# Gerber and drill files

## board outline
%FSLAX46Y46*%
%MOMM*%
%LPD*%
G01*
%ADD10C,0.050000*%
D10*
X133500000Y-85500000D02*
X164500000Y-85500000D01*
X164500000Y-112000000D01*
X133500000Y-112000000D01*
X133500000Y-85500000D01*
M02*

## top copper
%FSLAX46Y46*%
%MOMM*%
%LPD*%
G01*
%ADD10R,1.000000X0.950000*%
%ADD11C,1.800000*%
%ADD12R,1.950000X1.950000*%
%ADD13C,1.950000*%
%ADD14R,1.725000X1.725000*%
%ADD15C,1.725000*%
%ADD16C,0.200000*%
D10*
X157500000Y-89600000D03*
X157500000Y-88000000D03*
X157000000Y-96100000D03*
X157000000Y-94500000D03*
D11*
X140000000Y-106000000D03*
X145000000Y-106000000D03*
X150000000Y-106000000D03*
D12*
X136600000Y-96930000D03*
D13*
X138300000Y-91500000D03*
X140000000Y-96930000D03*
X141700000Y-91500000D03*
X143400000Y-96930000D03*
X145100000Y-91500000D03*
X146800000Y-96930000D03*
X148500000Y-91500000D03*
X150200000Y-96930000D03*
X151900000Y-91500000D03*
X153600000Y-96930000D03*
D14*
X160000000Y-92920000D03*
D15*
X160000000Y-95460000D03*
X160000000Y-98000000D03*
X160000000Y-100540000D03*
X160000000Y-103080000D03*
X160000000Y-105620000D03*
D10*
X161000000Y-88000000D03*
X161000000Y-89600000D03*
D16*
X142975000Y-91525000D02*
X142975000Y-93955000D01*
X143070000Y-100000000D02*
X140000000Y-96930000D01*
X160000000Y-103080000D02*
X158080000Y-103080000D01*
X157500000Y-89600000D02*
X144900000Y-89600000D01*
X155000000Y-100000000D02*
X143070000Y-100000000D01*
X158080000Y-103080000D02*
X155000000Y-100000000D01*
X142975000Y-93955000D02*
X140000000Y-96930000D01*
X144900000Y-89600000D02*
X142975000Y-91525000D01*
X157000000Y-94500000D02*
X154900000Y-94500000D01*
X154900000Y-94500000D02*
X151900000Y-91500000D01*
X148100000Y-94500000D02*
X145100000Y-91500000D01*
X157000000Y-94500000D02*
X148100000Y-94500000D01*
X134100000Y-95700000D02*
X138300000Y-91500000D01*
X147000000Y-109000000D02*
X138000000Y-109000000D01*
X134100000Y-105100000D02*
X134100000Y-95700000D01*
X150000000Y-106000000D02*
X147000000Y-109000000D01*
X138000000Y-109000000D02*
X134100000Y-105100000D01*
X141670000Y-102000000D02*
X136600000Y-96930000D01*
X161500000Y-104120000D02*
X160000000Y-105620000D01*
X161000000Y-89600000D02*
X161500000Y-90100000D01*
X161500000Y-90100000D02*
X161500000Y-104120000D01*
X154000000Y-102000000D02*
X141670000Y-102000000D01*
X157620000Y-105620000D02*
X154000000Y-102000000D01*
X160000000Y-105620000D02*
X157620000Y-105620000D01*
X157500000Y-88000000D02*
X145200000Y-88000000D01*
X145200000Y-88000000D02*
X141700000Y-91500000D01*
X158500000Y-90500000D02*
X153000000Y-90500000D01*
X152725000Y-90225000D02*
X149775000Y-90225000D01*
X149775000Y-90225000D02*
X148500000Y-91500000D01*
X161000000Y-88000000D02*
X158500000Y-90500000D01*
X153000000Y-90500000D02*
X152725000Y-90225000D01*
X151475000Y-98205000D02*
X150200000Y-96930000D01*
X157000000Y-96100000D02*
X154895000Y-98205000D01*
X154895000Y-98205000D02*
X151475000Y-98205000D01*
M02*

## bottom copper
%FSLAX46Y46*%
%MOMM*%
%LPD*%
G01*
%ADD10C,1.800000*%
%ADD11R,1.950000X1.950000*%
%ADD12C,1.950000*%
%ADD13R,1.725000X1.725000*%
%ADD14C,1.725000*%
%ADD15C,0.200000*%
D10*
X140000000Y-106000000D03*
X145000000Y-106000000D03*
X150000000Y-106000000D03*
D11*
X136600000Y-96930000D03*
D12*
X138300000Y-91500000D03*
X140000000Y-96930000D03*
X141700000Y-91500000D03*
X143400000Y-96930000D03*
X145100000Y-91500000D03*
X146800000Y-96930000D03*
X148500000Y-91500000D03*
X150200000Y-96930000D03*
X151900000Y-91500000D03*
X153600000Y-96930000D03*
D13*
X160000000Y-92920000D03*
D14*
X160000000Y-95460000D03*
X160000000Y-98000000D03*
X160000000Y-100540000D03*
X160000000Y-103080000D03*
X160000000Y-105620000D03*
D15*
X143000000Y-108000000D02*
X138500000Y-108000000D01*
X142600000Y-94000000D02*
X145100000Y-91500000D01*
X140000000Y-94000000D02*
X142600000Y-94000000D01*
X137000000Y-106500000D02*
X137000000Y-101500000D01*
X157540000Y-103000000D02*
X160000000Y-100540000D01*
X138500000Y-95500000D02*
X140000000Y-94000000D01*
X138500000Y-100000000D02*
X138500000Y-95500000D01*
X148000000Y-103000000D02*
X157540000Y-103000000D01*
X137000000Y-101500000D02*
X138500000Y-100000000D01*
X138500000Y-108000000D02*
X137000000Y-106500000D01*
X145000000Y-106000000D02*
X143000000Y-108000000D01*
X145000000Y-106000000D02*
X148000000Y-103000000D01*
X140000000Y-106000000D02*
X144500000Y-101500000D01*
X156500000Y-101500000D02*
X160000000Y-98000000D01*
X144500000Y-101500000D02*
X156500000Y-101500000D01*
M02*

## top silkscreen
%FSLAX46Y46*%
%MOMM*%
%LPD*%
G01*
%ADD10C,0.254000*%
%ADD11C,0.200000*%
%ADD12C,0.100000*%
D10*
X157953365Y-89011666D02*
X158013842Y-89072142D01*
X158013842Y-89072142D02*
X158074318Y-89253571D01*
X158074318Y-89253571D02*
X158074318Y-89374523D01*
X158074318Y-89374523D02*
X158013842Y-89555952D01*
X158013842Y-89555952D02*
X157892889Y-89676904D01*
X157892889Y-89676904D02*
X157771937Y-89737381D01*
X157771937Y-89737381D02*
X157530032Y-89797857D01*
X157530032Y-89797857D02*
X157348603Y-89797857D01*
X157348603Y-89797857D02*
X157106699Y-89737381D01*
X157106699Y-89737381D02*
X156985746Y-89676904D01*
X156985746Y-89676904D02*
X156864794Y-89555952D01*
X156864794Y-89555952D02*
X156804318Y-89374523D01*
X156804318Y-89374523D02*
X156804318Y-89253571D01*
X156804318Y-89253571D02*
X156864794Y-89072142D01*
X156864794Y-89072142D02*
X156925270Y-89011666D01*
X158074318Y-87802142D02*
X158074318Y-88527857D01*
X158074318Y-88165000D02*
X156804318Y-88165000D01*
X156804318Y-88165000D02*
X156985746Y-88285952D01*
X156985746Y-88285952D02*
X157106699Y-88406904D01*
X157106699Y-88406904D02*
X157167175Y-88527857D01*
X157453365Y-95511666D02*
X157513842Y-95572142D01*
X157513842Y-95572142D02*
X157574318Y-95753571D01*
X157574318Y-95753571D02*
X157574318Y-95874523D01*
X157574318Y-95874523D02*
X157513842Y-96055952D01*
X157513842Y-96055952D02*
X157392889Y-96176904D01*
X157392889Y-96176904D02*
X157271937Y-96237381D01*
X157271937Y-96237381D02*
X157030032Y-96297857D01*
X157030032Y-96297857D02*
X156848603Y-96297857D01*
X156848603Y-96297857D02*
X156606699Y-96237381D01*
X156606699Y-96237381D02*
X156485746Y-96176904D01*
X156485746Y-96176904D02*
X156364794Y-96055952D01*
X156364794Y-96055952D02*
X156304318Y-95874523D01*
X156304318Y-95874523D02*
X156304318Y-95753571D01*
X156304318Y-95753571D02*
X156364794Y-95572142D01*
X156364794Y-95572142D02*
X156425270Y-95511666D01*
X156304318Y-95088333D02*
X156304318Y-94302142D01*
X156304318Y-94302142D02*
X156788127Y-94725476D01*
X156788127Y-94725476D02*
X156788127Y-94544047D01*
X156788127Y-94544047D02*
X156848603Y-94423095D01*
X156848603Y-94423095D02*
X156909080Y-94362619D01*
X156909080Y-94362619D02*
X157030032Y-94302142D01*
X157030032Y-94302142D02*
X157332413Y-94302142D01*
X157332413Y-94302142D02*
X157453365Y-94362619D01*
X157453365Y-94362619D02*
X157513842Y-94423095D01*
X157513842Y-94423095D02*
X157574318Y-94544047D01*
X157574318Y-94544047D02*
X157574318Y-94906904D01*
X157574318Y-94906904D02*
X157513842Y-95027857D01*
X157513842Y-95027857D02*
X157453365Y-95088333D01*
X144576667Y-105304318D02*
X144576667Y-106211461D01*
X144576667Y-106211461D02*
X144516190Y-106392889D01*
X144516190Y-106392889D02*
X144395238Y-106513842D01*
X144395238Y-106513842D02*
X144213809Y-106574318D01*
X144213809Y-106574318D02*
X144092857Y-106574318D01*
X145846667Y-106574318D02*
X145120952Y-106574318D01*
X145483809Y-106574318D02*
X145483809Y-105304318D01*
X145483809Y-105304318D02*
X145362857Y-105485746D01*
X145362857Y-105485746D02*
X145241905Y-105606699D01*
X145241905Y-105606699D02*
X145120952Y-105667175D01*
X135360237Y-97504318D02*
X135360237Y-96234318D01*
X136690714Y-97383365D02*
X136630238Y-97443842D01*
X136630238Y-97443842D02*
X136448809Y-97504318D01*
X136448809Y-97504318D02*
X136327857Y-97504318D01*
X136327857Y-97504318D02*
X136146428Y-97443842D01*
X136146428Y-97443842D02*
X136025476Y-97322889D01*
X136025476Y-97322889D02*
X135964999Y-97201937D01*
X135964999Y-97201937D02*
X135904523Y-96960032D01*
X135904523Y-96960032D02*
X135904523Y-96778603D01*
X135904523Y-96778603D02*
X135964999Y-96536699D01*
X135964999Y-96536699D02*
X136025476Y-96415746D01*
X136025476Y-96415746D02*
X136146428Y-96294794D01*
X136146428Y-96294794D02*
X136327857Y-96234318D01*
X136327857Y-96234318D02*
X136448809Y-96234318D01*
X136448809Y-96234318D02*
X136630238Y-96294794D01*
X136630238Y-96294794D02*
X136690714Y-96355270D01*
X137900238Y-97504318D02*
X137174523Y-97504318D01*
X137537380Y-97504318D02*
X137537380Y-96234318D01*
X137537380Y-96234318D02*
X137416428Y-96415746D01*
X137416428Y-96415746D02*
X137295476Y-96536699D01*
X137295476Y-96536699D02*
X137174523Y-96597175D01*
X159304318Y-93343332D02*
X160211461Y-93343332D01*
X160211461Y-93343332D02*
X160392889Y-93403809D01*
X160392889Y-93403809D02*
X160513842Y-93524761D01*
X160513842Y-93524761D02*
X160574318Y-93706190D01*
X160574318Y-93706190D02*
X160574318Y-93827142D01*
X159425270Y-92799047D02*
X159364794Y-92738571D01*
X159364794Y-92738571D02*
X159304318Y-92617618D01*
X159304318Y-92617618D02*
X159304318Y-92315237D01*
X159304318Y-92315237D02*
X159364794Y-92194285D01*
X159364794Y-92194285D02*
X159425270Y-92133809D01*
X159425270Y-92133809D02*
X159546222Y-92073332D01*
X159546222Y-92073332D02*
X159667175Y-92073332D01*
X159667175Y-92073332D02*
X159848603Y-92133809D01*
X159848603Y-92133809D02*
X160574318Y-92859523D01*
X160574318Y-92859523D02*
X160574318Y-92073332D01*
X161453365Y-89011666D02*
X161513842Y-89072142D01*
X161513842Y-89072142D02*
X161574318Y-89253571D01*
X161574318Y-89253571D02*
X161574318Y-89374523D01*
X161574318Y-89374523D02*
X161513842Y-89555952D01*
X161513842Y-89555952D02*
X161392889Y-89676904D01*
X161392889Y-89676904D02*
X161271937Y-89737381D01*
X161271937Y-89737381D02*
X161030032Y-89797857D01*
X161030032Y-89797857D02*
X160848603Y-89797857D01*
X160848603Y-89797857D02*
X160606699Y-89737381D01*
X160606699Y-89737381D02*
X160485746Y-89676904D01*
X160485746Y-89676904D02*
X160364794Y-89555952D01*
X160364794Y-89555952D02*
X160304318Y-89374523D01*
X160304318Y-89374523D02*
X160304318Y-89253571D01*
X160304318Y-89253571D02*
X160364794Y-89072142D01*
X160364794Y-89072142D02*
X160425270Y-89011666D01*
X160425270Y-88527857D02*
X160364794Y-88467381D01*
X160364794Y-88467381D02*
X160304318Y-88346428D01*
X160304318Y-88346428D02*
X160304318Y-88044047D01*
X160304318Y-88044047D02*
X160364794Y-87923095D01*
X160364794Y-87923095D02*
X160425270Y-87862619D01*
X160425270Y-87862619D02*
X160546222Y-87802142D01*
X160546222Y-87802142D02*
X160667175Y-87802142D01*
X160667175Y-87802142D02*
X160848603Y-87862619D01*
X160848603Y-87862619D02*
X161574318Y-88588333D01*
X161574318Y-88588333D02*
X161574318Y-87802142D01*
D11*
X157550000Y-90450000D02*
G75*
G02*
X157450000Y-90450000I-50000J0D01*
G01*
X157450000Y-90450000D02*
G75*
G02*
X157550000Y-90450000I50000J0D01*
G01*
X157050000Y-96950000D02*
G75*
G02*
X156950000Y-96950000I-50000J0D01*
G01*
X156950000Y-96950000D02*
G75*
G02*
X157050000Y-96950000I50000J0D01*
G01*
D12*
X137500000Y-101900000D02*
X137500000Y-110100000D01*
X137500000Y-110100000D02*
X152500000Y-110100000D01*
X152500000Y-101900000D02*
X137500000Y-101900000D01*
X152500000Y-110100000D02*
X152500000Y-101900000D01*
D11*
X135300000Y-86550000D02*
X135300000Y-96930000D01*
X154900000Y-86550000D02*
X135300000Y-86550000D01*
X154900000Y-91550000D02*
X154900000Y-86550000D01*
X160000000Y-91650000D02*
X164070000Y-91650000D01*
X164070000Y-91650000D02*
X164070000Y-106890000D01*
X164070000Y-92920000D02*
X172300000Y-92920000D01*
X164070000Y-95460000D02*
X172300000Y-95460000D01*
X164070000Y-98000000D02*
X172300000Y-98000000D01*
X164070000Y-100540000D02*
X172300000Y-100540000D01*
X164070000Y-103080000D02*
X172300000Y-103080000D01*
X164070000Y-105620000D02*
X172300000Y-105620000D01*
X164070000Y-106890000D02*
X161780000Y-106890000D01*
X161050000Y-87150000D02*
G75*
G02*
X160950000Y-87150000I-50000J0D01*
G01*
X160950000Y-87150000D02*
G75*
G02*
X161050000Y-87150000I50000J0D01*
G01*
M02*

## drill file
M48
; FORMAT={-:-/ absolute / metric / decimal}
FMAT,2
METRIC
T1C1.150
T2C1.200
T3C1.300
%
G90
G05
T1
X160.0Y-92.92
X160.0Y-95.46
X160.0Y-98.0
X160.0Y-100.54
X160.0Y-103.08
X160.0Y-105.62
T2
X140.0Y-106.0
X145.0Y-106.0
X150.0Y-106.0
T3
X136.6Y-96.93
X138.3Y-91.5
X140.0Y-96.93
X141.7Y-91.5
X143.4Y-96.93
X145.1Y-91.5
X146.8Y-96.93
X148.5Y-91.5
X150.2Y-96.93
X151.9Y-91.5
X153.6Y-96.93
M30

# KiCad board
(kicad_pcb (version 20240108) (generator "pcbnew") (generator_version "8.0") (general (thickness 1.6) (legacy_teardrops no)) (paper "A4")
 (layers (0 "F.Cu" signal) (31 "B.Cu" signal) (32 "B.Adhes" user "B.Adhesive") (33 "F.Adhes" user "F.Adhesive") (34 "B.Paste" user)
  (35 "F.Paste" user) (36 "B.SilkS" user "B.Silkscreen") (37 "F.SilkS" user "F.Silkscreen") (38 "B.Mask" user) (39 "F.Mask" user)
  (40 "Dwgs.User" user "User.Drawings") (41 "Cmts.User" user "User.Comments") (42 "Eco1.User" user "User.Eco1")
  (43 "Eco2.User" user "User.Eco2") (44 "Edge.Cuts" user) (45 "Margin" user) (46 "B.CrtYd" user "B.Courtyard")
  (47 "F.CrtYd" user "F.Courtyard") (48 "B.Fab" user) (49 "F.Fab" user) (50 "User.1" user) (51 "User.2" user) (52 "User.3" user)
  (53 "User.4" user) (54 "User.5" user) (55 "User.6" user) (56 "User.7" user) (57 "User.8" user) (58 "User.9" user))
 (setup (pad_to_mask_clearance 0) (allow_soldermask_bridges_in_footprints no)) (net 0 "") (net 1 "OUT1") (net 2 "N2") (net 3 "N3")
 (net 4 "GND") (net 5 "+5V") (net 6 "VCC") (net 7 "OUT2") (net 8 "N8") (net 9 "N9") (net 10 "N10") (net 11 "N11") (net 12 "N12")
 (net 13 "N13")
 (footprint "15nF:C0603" (layer "F.Cu") (at 157.5 88.8 90)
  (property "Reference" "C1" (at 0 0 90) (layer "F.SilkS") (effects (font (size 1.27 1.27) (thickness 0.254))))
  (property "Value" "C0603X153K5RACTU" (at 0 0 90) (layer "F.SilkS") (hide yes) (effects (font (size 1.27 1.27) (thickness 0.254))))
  (fp_circle (center -1.65 0) (end -1.65 0.05) (stroke (width 0.2) (type solid)) (fill none) (layer "F.SilkS"))
  (pad "1" smd rect (at -0.8 0 90) (size 0.95 1) (layers "F.Cu" "F.Paste" "F.Mask") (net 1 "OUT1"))
  (pad "2" smd rect (at 0.8 0 90) (size 0.95 1) (layers "F.Cu" "F.Paste" "F.Mask") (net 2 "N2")))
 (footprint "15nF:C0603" (layer "F.Cu") (at 157 95.3 90)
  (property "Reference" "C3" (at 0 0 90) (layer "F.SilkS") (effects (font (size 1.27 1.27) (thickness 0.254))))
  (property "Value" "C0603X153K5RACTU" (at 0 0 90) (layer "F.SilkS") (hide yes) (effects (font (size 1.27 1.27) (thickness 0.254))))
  (fp_circle (center -1.65 0) (end -1.65 0.05) (stroke (width 0.2) (type solid)) (fill none) (layer "F.SilkS"))
  (pad "1" smd rect (at -0.8 0 90) (size 0.95 1) (layers "F.Cu" "F.Paste" "F.Mask") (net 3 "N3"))
  (pad "2" smd rect (at 0.8 0 90) (size 0.95 1) (layers "F.Cu" "F.Paste" "F.Mask") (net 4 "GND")))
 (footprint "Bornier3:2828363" (layer "F.Cu") (at 140 106)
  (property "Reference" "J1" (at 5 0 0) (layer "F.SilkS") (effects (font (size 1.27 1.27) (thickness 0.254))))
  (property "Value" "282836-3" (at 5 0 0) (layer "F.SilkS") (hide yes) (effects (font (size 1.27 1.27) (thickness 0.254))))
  (fp_line (start -2.5 -4.1) (end -2.5 4.1) (stroke (width 0.1) (type solid)) (layer "F.SilkS"))
  (fp_line (start -2.5 4.1) (end 12.5 4.1) (stroke (width 0.1) (type solid)) (layer "F.SilkS"))
  (fp_line (start 12.5 -4.1) (end -2.5 -4.1) (stroke (width 0.1) (type solid)) (layer "F.SilkS"))
  (fp_line (start 12.5 4.1) (end 12.5 -4.1) (stroke (width 0.1) (type solid)) (layer "F.SilkS"))
  (pad "1" thru_hole circle (at 0 0) (size 1.8 1.8) (drill 1.2) (layers "*.Cu" "*.Mask") (remove_unused_layers no) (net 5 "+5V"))
  (pad "2" thru_hole circle (at 5 0) (size 1.8 1.8) (drill 1.2) (layers "*.Cu" "*.Mask") (remove_unused_layers no) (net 4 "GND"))
  (pad "3" thru_hole circle (at 10 0) (size 1.8 1.8) (drill 1.2) (layers "*.Cu" "*.Mask") (remove_unused_layers no) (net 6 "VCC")))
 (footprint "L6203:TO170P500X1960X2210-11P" (layer "F.Cu") (at 136.6 96.93)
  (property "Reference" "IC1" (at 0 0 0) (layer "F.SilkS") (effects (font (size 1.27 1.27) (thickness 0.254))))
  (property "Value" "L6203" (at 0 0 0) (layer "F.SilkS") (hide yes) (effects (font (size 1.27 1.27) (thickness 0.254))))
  (fp_line (start -1.3 -10.38) (end -1.3 0) (stroke (width 0.2) (type solid)) (layer "F.SilkS"))
  (fp_line (start 18.3 -10.38) (end -1.3 -10.38) (stroke (width 0.2) (type solid)) (layer "F.SilkS"))
  (fp_line (start 18.3 -5.38) (end 18.3 -10.38) (stroke (width 0.2) (type solid)) (layer "F.SilkS"))
  (pad "1" thru_hole rect (at 0 0) (size 1.95 1.95) (drill 1.3) (layers "*.Cu" "*.Mask") (remove_unused_layers no) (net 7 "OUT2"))
  (pad "2" thru_hole circle (at 1.7 -5.43) (size 1.95 1.95) (drill 1.3) (layers "*.Cu" "*.Mask") (remove_unused_layers no) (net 6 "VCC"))
  (pad "3" thru_hole circle (at 3.4 0) (size 1.95 1.95) (drill 1.3) (layers "*.Cu" "*.Mask") (remove_unused_layers no) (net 1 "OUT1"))
  (pad "4" thru_hole circle (at 5.1 -5.43) (size 1.95 1.95) (drill 1.3) (layers "*.Cu" "*.Mask") (remove_unused_layers no) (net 2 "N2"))
  (pad "5" thru_hole circle (at 6.8 0) (size 1.95 1.95) (drill 1.3) (layers "*.Cu" "*.Mask") (remove_unused_layers no) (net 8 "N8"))
  (pad "6" thru_hole circle (at 8.5 -5.43) (size 1.95 1.95) (drill 1.3) (layers "*.Cu" "*.Mask") (remove_unused_layers no) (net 4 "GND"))
  (pad "7" thru_hole circle (at 10.2 0) (size 1.95 1.95) (drill 1.3) (layers "*.Cu" "*.Mask") (remove_unused_layers no) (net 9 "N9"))
  (pad "8" thru_hole circle (at 11.9 -5.43) (size 1.95 1.95) (drill 1.3) (layers "*.Cu" "*.Mask") (remove_unused_layers no) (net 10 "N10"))
  (pad "9" thru_hole circle (at 13.6 0) (size 1.95 1.95) (drill 1.3) (layers "*.Cu" "*.Mask") (remove_unused_layers no) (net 3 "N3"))
  (pad "10" thru_hole circle (at 15.3 -5.43) (size 1.95 1.95) (drill 1.3) (layers "*.Cu" "*.Mask") (remove_unused_layers no) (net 4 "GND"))
  (pad "11" thru_hole circle (at 17 0) (size 1.95 1.95) (drill 1.3) (layers "*.Cu" "*.Mask") (remove_unused_layers no) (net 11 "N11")))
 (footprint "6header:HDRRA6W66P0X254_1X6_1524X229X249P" (layer "F.Cu") (at 160 92.92 -90)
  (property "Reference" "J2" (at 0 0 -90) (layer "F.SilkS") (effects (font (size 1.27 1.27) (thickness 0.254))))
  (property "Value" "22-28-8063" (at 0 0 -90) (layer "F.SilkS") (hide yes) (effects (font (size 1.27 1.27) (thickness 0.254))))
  (fp_line (start -1.27 0) (end -1.27 -4.07) (stroke (width 0.2) (type solid)) (layer "F.SilkS"))
  (fp_line (start -1.27 -4.07) (end 13.97 -4.07) (stroke (width 0.2) (type solid)) (layer "F.SilkS"))
  (fp_line (start 0 -4.07) (end 0 -12.3) (stroke (width 0.2) (type solid)) (layer "F.SilkS"))
  (fp_line (start 2.54 -4.07) (end 2.54 -12.3) (stroke (width 0.2) (type solid)) (layer "F.SilkS"))
  (fp_line (start 5.08 -4.07) (end 5.08 -12.3) (stroke (width 0.2) (type solid)) (layer "F.SilkS"))
  (fp_line (start 7.62 -4.07) (end 7.62 -12.3) (stroke (width 0.2) (type solid)) (layer "F.SilkS"))
  (fp_line (start 10.16 -4.07) (end 10.16 -12.3) (stroke (width 0.2) (type solid)) (layer "F.SilkS"))
  (fp_line (start 12.7 -4.07) (end 12.7 -12.3) (stroke (width 0.2) (type solid)) (layer "F.SilkS"))
  (fp_line (start 13.97 -4.07) (end 13.97 -1.78) (stroke (width 0.2) (type solid)) (layer "F.SilkS"))
  (pad "1" thru_hole rect (at 0 0 270) (size 1.725 1.725) (drill 1.15) (layers "*.Cu" "*.Mask") (remove_unused_layers no) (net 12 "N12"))
  (pad "2" thru_hole circle (at 2.54 0 270) (size 1.725 1.725) (drill 1.15) (layers "*.Cu" "*.Mask") (remove_unused_layers no)
   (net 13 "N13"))
  (pad "3" thru_hole circle (at 5.08 0 270) (size 1.725 1.725) (drill 1.15) (layers "*.Cu" "*.Mask") (remove_unused_layers no) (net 5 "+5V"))
  (pad "4" thru_hole circle (at 7.62 0 270) (size 1.725 1.725) (drill 1.15) (layers "*.Cu" "*.Mask") (remove_unused_layers no) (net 4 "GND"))
  (pad "5" thru_hole circle (at 10.16 0 270) (size 1.725 1.725) (drill 1.15) (layers "*.Cu" "*.Mask") (remove_unused_layers no)
   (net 1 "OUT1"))
  (pad "6" thru_hole circle (at 12.7 0 270) (size 1.725 1.725) (drill 1.15) (layers "*.Cu" "*.Mask") (remove_unused_layers no)
   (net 7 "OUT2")))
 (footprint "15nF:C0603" (layer "F.Cu") (at 161 88.8 -90)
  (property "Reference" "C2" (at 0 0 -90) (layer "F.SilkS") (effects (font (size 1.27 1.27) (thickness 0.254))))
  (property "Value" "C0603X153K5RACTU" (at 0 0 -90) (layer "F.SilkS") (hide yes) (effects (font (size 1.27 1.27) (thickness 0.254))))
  (fp_circle (center -1.65 0) (end -1.65 0.05) (stroke (width 0.2) (type solid)) (fill none) (layer "F.SilkS"))
  (pad "1" smd rect (at -0.8 0 270) (size 0.95 1) (layers "F.Cu" "F.Paste" "F.Mask") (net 10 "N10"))
  (pad "2" smd rect (at 0.8 0 270) (size 0.95 1) (layers "F.Cu" "F.Paste" "F.Mask") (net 7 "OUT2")))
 (gr_rect (start 133.5 85.5) (end 164.5 112) (stroke (width 0.05) (type default)) (fill none) (layer "Edge.Cuts"))
 (segment (start 142.975 91.525) (end 142.975 93.955) (width 0.2) (layer "F.Cu") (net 1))
 (segment (start 143.07 100) (end 140 96.93) (width 0.2) (layer "F.Cu") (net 1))
 (segment (start 160 103.08) (end 158.08 103.08) (width 0.2) (layer "F.Cu") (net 1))
 (segment (start 157.5 89.6) (end 144.9 89.6) (width 0.2) (layer "F.Cu") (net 1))
 (segment (start 155 100) (end 143.07 100) (width 0.2) (layer "F.Cu") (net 1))
 (segment (start 158.08 103.08) (end 155 100) (width 0.2) (layer "F.Cu") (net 1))
 (segment (start 142.975 93.955) (end 140 96.93) (width 0.2) (layer "F.Cu") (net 1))
 (segment (start 144.9 89.6) (end 142.975 91.525) (width 0.2) (layer "F.Cu") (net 1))
 (segment (start 157 94.5) (end 154.9 94.5) (width 0.2) (layer "F.Cu") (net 4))
 (segment (start 154.9 94.5) (end 151.9 91.5) (width 0.2) (layer "F.Cu") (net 4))
 (segment (start 148.1 94.5) (end 145.1 91.5) (width 0.2) (layer "F.Cu") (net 4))
 (segment (start 157 94.5) (end 148.1 94.5) (width 0.2) (layer "F.Cu") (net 4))
 (segment (start 143 108) (end 138.5 108) (width 0.2) (layer "B.Cu") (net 4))
 (segment (start 142.6 94) (end 145.1 91.5) (width 0.2) (layer "B.Cu") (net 4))
 (segment (start 140 94) (end 142.6 94) (width 0.2) (layer "B.Cu") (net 4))
 (segment (start 137 106.5) (end 137 101.5) (width 0.2) (layer "B.Cu") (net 4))
 (segment (start 157.54 103) (end 160 100.54) (width 0.2) (layer "B.Cu") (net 4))
 (segment (start 138.5 95.5) (end 140 94) (width 0.2) (layer "B.Cu") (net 4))
 (segment (start 138.5 100) (end 138.5 95.5) (width 0.2) (layer "B.Cu") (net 4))
 (segment (start 148 103) (end 157.54 103) (width 0.2) (layer "B.Cu") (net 4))
 (segment (start 137 101.5) (end 138.5 100) (width 0.2) (layer "B.Cu") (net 4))
 (segment (start 138.5 108) (end 137 106.5) (width 0.2) (layer "B.Cu") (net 4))
 (segment (start 145 106) (end 143 108) (width 0.2) (layer "B.Cu") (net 4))
 (segment (start 145 106) (end 148 103) (width 0.2) (layer "B.Cu") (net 4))
 (segment (start 134.1 95.7) (end 138.3 91.5) (width 0.2) (layer "F.Cu") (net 6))
 (segment (start 147 109) (end 138 109) (width 0.2) (layer "F.Cu") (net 6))
 (segment (start 134.1 105.1) (end 134.1 95.7) (width 0.2) (layer "F.Cu") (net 6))
 (segment (start 150 106) (end 147 109) (width 0.2) (layer "F.Cu") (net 6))
 (segment (start 138 109) (end 134.1 105.1) (width 0.2) (layer "F.Cu") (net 6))
 (segment (start 141.67 102) (end 136.6 96.93) (width 0.2) (layer "F.Cu") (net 7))
 (segment (start 161.5 104.12) (end 160 105.62) (width 0.2) (layer "F.Cu") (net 7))
 (segment (start 161 89.6) (end 161.5 90.1) (width 0.2) (layer "F.Cu") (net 7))
 (segment (start 161.5 90.1) (end 161.5 104.12) (width 0.2) (layer "F.Cu") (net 7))
 (segment (start 154 102) (end 141.67 102) (width 0.2) (layer "F.Cu") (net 7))
 (segment (start 157.62 105.62) (end 154 102) (width 0.2) (layer "F.Cu") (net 7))
 (segment (start 160 105.62) (end 157.62 105.62) (width 0.2) (layer "F.Cu") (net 7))
 (segment (start 140 106) (end 144.5 101.5) (width 0.2) (layer "B.Cu") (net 5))
 (segment (start 156.5 101.5) (end 160 98) (width 0.2) (layer "B.Cu") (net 5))
 (segment (start 144.5 101.5) (end 156.5 101.5) (width 0.2) (layer "B.Cu") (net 5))
 (segment (start 157.5 88) (end 145.2 88) (width 0.2) (layer "F.Cu") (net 2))
 (segment (start 145.2 88) (end 141.7 91.5) (width 0.2) (layer "F.Cu") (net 2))
 (segment (start 158.5 90.5) (end 153 90.5) (width 0.2) (layer "F.Cu") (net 10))
 (segment (start 152.725 90.225) (end 149.775 90.225) (width 0.2) (layer "F.Cu") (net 10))
 (segment (start 149.775 90.225) (end 148.5 91.5) (width 0.2) (layer "F.Cu") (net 10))
 (segment (start 161 88) (end 158.5 90.5) (width 0.2) (layer "F.Cu") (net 10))
 (segment (start 153 90.5) (end 152.725 90.225) (width 0.2) (layer "F.Cu") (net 10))
 (segment (start 151.475 98.205) (end 150.2 96.93) (width 0.2) (layer "F.Cu") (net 3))
 (segment (start 157 96.1) (end 154.895 98.205) (width 0.2) (layer "F.Cu") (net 3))
 (segment (start 154.895 98.205) (end 151.475 98.205) (width 0.2) (layer "F.Cu") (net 3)))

